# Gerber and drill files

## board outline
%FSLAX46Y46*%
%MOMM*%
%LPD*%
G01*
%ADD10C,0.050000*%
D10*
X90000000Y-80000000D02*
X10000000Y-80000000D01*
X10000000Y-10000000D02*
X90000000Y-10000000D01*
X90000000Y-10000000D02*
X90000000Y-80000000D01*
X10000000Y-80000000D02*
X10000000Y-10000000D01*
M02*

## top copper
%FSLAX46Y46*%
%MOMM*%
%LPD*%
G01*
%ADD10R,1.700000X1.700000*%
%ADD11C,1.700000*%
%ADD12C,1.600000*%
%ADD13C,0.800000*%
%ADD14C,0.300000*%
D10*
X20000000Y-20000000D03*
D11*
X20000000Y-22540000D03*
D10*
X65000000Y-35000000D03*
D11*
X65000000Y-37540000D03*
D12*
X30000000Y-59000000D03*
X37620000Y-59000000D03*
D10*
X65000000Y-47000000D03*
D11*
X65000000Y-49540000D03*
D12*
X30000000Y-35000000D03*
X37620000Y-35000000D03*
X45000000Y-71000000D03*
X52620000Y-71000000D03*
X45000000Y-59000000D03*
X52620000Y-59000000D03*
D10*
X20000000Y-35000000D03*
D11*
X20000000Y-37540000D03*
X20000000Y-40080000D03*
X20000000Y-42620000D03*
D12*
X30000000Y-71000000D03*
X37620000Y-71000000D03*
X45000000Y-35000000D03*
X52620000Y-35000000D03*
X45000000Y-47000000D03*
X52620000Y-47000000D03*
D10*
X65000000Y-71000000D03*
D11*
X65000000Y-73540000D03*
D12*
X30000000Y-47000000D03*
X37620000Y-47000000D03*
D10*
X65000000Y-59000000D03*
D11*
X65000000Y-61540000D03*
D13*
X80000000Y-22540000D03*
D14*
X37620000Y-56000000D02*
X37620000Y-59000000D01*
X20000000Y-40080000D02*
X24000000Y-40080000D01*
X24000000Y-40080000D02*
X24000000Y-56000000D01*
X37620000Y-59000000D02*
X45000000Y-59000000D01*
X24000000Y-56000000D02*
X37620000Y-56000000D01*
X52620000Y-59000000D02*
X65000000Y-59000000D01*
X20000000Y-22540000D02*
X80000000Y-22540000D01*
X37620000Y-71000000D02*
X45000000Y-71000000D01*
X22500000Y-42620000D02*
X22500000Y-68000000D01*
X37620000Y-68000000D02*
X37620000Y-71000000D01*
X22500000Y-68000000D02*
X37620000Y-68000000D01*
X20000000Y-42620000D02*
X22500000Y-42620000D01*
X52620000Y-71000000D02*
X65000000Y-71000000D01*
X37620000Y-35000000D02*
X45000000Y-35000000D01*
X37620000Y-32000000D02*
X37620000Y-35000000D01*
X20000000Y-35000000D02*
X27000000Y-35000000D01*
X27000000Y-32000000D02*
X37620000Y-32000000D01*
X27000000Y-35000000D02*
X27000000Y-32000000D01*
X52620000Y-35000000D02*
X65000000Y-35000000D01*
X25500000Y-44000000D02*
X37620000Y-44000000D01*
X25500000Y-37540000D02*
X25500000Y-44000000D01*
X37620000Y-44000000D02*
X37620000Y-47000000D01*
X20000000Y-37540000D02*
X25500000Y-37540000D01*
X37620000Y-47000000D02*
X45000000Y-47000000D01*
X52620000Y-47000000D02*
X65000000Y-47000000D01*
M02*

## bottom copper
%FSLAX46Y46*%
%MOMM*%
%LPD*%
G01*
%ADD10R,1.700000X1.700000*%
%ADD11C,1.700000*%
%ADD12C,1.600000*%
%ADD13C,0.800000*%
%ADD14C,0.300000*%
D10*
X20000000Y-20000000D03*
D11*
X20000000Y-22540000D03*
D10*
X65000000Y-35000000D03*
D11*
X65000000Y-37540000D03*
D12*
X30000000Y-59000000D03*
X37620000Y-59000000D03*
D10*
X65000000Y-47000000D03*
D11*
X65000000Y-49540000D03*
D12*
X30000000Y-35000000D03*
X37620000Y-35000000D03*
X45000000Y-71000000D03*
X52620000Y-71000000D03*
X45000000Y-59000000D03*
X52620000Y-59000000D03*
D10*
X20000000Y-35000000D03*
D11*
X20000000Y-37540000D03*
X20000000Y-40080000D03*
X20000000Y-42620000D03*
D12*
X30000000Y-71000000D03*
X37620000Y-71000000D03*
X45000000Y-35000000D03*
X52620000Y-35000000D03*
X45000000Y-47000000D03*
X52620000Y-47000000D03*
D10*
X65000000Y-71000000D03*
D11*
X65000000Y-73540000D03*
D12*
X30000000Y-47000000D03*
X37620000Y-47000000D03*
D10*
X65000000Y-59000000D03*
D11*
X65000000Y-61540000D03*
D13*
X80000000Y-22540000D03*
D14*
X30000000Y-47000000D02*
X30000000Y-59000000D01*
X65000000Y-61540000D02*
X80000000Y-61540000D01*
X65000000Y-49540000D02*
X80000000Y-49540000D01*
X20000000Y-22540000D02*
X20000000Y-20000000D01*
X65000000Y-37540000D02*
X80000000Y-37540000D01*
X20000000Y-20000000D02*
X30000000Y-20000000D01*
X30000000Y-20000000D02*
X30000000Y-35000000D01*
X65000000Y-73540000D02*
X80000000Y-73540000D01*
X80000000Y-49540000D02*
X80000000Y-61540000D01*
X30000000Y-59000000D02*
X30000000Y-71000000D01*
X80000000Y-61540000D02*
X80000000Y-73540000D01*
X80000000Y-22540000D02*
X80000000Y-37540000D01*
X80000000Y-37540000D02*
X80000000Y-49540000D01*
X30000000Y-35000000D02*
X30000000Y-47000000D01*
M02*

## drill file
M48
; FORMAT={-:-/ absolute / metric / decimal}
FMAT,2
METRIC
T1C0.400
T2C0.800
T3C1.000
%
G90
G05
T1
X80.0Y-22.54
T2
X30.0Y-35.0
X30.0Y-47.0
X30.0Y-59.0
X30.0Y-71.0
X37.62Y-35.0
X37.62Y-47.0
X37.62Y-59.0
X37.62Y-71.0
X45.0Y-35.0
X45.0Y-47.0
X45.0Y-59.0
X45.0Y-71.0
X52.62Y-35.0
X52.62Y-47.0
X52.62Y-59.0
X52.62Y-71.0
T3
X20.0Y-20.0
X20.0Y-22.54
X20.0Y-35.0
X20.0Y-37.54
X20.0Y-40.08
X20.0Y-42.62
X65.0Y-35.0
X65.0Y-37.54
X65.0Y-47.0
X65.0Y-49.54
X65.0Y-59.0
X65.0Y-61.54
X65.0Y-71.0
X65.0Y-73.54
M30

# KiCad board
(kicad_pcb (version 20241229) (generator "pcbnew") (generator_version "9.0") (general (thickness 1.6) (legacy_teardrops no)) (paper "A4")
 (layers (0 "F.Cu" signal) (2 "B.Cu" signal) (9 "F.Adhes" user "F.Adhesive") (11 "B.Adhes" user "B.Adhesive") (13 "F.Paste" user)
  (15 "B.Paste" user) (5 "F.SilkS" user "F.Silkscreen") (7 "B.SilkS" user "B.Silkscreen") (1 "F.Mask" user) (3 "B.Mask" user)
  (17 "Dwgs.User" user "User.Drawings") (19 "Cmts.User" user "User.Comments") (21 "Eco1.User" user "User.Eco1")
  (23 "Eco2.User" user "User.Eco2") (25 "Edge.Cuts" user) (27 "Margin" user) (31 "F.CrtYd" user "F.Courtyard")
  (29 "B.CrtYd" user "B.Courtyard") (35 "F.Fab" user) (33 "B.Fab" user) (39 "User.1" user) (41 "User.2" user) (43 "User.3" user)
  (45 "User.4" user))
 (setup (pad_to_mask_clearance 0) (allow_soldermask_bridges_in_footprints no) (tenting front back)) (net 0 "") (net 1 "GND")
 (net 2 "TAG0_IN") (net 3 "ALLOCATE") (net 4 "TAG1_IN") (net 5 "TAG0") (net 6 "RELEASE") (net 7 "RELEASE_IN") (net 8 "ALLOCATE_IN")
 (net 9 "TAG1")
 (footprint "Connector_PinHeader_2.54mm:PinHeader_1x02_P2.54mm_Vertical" (layer "F.Cu") (at 20 20)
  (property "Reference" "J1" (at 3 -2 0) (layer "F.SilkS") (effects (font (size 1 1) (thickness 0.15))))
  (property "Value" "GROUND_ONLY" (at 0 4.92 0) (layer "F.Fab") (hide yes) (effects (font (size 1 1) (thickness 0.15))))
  (pad "1" thru_hole rect (at 0 0) (size 1.7 1.7) (drill 1) (layers "*.Cu" "*.Mask") (remove_unused_layers no) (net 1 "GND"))
  (pad "2" thru_hole circle (at 0 2.54) (size 1.7 1.7) (drill 1) (layers "*.Cu" "*.Mask") (remove_unused_layers no) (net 1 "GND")))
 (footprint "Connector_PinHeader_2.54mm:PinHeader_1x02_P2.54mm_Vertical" (layer "F.Cu") (at 65 35)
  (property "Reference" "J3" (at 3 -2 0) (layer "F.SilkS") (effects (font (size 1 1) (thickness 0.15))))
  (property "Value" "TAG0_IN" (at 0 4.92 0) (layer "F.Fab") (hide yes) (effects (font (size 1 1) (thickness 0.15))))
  (pad "1" thru_hole rect (at 0 0) (size 1.7 1.7) (drill 1) (layers "*.Cu" "*.Mask") (remove_unused_layers no) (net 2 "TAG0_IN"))
  (pad "2" thru_hole circle (at 0 2.54) (size 1.7 1.7) (drill 1) (layers "*.Cu" "*.Mask") (remove_unused_layers no) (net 1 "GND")))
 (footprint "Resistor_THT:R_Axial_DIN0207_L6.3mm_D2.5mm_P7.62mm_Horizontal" (layer "F.Cu") (at 30 59)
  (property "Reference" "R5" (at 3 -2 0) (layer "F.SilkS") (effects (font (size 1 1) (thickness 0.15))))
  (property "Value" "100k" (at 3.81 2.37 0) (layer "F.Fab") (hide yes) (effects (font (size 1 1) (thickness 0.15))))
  (pad "1" thru_hole circle (at 0 0) (size 1.6 1.6) (drill 0.8) (layers "*.Cu" "*.Mask") (remove_unused_layers no) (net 1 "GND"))
  (pad "2" thru_hole circle (at 7.62 0) (size 1.6 1.6) (drill 0.8) (layers "*.Cu" "*.Mask") (remove_unused_layers no) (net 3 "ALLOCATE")))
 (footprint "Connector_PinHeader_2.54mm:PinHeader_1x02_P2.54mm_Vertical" (layer "F.Cu") (at 65 47)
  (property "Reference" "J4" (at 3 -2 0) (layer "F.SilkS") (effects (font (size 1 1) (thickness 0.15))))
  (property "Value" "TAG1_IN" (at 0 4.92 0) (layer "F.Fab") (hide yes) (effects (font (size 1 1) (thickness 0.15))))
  (pad "1" thru_hole rect (at 0 0) (size 1.7 1.7) (drill 1) (layers "*.Cu" "*.Mask") (remove_unused_layers no) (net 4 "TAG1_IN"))
  (pad "2" thru_hole circle (at 0 2.54) (size 1.7 1.7) (drill 1) (layers "*.Cu" "*.Mask") (remove_unused_layers no) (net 1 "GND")))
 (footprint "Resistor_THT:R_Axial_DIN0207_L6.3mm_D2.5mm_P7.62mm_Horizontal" (layer "F.Cu") (at 30 35)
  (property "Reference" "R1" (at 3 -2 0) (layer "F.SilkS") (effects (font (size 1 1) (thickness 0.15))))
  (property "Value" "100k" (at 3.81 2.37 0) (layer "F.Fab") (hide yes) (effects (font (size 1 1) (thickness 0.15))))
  (pad "1" thru_hole circle (at 0 0) (size 1.6 1.6) (drill 0.8) (layers "*.Cu" "*.Mask") (remove_unused_layers no) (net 1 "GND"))
  (pad "2" thru_hole circle (at 7.62 0) (size 1.6 1.6) (drill 0.8) (layers "*.Cu" "*.Mask") (remove_unused_layers no) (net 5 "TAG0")))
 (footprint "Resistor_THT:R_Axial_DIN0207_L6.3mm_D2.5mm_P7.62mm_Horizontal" (layer "F.Cu") (at 45 71)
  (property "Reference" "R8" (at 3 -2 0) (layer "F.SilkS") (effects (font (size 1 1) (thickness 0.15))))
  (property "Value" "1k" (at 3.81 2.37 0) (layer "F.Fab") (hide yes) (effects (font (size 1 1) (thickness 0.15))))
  (pad "1" thru_hole circle (at 0 0) (size 1.6 1.6) (drill 0.8) (layers "*.Cu" "*.Mask") (remove_unused_layers no) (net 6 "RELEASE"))
  (pad "2" thru_hole circle (at 7.62 0) (size 1.6 1.6) (drill 0.8) (layers "*.Cu" "*.Mask") (remove_unused_layers no) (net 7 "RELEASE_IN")))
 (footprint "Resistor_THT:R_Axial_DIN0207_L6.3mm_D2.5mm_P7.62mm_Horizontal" (layer "F.Cu") (at 45 59)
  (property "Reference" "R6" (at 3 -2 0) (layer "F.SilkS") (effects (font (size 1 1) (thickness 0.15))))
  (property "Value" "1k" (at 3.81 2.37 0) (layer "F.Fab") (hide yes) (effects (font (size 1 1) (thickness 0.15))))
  (pad "1" thru_hole circle (at 0 0) (size 1.6 1.6) (drill 0.8) (layers "*.Cu" "*.Mask") (remove_unused_layers no) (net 3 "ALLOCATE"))
  (pad "2" thru_hole circle (at 7.62 0) (size 1.6 1.6) (drill 0.8) (layers "*.Cu" "*.Mask") (remove_unused_layers no) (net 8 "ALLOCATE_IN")))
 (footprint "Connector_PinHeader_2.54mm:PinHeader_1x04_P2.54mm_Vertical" (layer "F.Cu") (at 20 35)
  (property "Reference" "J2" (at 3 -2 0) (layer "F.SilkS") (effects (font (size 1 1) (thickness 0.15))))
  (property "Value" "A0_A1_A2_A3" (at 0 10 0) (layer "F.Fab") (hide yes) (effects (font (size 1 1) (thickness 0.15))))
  (pad "1" thru_hole rect (at 0 0) (size 1.7 1.7) (drill 1) (layers "*.Cu" "*.Mask") (remove_unused_layers no) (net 5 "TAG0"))
  (pad "2" thru_hole circle (at 0 2.54) (size 1.7 1.7) (drill 1) (layers "*.Cu" "*.Mask") (remove_unused_layers no) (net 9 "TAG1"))
  (pad "3" thru_hole circle (at 0 5.08) (size 1.7 1.7) (drill 1) (layers "*.Cu" "*.Mask") (remove_unused_layers no) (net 3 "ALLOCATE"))
  (pad "4" thru_hole circle (at 0 7.62) (size 1.7 1.7) (drill 1) (layers "*.Cu" "*.Mask") (remove_unused_layers no) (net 6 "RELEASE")))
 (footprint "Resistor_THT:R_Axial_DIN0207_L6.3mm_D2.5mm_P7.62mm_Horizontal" (layer "F.Cu") (at 30 71)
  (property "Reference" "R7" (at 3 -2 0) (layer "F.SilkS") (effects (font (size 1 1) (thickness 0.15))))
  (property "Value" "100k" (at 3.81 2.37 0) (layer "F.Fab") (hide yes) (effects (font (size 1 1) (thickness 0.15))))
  (pad "1" thru_hole circle (at 0 0) (size 1.6 1.6) (drill 0.8) (layers "*.Cu" "*.Mask") (remove_unused_layers no) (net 1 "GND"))
  (pad "2" thru_hole circle (at 7.62 0) (size 1.6 1.6) (drill 0.8) (layers "*.Cu" "*.Mask") (remove_unused_layers no) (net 6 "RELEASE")))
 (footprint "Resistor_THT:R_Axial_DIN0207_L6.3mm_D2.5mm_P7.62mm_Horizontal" (layer "F.Cu") (at 45 35)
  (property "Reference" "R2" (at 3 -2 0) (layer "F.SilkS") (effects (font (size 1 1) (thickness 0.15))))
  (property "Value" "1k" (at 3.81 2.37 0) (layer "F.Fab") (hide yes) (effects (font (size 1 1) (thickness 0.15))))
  (pad "1" thru_hole circle (at 0 0) (size 1.6 1.6) (drill 0.8) (layers "*.Cu" "*.Mask") (remove_unused_layers no) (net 5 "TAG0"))
  (pad "2" thru_hole circle (at 7.62 0) (size 1.6 1.6) (drill 0.8) (layers "*.Cu" "*.Mask") (remove_unused_layers no) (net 2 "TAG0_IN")))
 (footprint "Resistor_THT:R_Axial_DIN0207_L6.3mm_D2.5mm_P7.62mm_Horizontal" (layer "F.Cu") (at 45 47)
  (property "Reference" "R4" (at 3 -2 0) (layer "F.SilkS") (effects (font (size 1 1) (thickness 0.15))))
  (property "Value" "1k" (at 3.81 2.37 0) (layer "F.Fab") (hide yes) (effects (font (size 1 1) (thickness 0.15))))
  (pad "1" thru_hole circle (at 0 0) (size 1.6 1.6) (drill 0.8) (layers "*.Cu" "*.Mask") (remove_unused_layers no) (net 9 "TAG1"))
  (pad "2" thru_hole circle (at 7.62 0) (size 1.6 1.6) (drill 0.8) (layers "*.Cu" "*.Mask") (remove_unused_layers no) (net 4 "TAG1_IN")))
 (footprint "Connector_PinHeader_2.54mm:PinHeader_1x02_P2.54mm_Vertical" (layer "F.Cu") (at 65 71)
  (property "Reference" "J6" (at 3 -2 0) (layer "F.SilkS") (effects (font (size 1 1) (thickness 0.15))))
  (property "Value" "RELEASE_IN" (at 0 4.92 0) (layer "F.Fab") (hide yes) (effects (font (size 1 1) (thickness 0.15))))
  (pad "1" thru_hole rect (at 0 0) (size 1.7 1.7) (drill 1) (layers "*.Cu" "*.Mask") (remove_unused_layers no) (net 7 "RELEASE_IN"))
  (pad "2" thru_hole circle (at 0 2.54) (size 1.7 1.7) (drill 1) (layers "*.Cu" "*.Mask") (remove_unused_layers no) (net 1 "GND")))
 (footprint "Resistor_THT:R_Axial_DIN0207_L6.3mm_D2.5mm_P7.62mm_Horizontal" (layer "F.Cu") (at 30 47)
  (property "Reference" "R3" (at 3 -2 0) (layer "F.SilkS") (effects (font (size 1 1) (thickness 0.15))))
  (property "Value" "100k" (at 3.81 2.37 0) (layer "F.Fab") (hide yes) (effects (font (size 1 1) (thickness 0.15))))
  (pad "1" thru_hole circle (at 0 0) (size 1.6 1.6) (drill 0.8) (layers "*.Cu" "*.Mask") (remove_unused_layers no) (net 1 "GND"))
  (pad "2" thru_hole circle (at 7.62 0) (size 1.6 1.6) (drill 0.8) (layers "*.Cu" "*.Mask") (remove_unused_layers no) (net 9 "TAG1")))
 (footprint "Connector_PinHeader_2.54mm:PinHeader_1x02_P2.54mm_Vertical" (layer "F.Cu") (at 65 59)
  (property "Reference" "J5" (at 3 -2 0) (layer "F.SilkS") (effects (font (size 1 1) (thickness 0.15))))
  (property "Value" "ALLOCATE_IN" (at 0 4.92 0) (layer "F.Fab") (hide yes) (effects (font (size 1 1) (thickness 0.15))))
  (pad "1" thru_hole rect (at 0 0) (size 1.7 1.7) (drill 1) (layers "*.Cu" "*.Mask") (remove_unused_layers no) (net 8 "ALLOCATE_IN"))
  (pad "2" thru_hole circle (at 0 2.54) (size 1.7 1.7) (drill 1) (layers "*.Cu" "*.Mask") (remove_unused_layers no) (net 1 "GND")))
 (gr_line (start 90 80) (end 10 80) (stroke (width 0.05) (type default)) (layer "Edge.Cuts"))
 (gr_line (start 10 10) (end 90 10) (stroke (width 0.05) (type default)) (layer "Edge.Cuts"))
 (gr_line (start 90 10) (end 90 80) (stroke (width 0.05) (type default)) (layer "Edge.Cuts"))
 (gr_line (start 10 80) (end 10 10) (stroke (width 0.05) (type default)) (layer "Edge.Cuts"))
 (segment (start 37.62 56) (end 37.62 59) (width 0.3) (layer "F.Cu") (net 3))
 (segment (start 20 40.08) (end 24 40.08) (width 0.3) (layer "F.Cu") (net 3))
 (segment (start 24 40.08) (end 24 56) (width 0.3) (layer "F.Cu") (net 3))
 (segment (start 37.62 59) (end 45 59) (width 0.3) (layer "F.Cu") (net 3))
 (segment (start 24 56) (end 37.62 56) (width 0.3) (layer "F.Cu") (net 3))
 (segment (start 52.62 59) (end 65 59) (width 0.3) (layer "F.Cu") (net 8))
 (segment (start 20 22.54) (end 80 22.54) (width 0.3) (layer "F.Cu") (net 1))
 (via (at 80 22.54) (size 0.8) (drill 0.4) (layers "F.Cu" "B.Cu") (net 1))
 (segment (start 30 47) (end 30 59) (width 0.3) (layer "B.Cu") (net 1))
 (segment (start 65 61.54) (end 80 61.54) (width 0.3) (layer "B.Cu") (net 1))
 (segment (start 65 49.54) (end 80 49.54) (width 0.3) (layer "B.Cu") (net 1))
 (segment (start 20 22.54) (end 20 20) (width 0.3) (layer "B.Cu") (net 1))
 (segment (start 65 37.54) (end 80 37.54) (width 0.3) (layer "B.Cu") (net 1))
 (segment (start 20 20) (end 30 20) (width 0.3) (layer "B.Cu") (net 1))
 (segment (start 30 20) (end 30 35) (width 0.3) (layer "B.Cu") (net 1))
 (segment (start 65 73.54) (end 80 73.54) (width 0.3) (layer "B.Cu") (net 1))
 (segment (start 80 49.54) (end 80 61.54) (width 0.3) (layer "B.Cu") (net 1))
 (segment (start 30 59) (end 30 71) (width 0.3) (layer "B.Cu") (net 1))
 (segment (start 80 61.54) (end 80 73.54) (width 0.3) (layer "B.Cu") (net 1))
 (segment (start 80 22.54) (end 80 37.54) (width 0.3) (layer "B.Cu") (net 1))
 (segment (start 80 37.54) (end 80 49.54) (width 0.3) (layer "B.Cu") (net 1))
 (segment (start 30 35) (end 30 47) (width 0.3) (layer "B.Cu") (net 1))
 (segment (start 37.62 71) (end 45 71) (width 0.3) (layer "F.Cu") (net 6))
 (segment (start 22.5 42.62) (end 22.5 68) (width 0.3) (layer "F.Cu") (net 6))
 (segment (start 37.62 68) (end 37.62 71) (width 0.3) (layer "F.Cu") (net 6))
 (segment (start 22.5 68) (end 37.62 68) (width 0.3) (layer "F.Cu") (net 6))
 (segment (start 20 42.62) (end 22.5 42.62) (width 0.3) (layer "F.Cu") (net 6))
 (segment (start 52.62 71) (end 65 71) (width 0.3) (layer "F.Cu") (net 7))
 (segment (start 37.62 35) (end 45 35) (width 0.3) (layer "F.Cu") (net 5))
 (segment (start 37.62 32) (end 37.62 35) (width 0.3) (layer "F.Cu") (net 5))
 (segment (start 20 35) (end 27 35) (width 0.3) (layer "F.Cu") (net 5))
 (segment (start 27 32) (end 37.62 32) (width 0.3) (layer "F.Cu") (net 5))
 (segment (start 27 35) (end 27 32) (width 0.3) (layer "F.Cu") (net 5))
 (segment (start 52.62 35) (end 65 35) (width 0.3) (layer "F.Cu") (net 2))
 (segment (start 25.5 44) (end 37.62 44) (width 0.3) (layer "F.Cu") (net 9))
 (segment (start 25.5 37.54) (end 25.5 44) (width 0.3) (layer "F.Cu") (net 9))
 (segment (start 37.62 44) (end 37.62 47) (width 0.3) (layer "F.Cu") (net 9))
 (segment (start 20 37.54) (end 25.5 37.54) (width 0.3) (layer "F.Cu") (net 9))
 (segment (start 37.62 47) (end 45 47) (width 0.3) (layer "F.Cu") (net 9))
 (segment (start 52.62 47) (end 65 47) (width 0.3) (layer "F.Cu") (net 4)))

